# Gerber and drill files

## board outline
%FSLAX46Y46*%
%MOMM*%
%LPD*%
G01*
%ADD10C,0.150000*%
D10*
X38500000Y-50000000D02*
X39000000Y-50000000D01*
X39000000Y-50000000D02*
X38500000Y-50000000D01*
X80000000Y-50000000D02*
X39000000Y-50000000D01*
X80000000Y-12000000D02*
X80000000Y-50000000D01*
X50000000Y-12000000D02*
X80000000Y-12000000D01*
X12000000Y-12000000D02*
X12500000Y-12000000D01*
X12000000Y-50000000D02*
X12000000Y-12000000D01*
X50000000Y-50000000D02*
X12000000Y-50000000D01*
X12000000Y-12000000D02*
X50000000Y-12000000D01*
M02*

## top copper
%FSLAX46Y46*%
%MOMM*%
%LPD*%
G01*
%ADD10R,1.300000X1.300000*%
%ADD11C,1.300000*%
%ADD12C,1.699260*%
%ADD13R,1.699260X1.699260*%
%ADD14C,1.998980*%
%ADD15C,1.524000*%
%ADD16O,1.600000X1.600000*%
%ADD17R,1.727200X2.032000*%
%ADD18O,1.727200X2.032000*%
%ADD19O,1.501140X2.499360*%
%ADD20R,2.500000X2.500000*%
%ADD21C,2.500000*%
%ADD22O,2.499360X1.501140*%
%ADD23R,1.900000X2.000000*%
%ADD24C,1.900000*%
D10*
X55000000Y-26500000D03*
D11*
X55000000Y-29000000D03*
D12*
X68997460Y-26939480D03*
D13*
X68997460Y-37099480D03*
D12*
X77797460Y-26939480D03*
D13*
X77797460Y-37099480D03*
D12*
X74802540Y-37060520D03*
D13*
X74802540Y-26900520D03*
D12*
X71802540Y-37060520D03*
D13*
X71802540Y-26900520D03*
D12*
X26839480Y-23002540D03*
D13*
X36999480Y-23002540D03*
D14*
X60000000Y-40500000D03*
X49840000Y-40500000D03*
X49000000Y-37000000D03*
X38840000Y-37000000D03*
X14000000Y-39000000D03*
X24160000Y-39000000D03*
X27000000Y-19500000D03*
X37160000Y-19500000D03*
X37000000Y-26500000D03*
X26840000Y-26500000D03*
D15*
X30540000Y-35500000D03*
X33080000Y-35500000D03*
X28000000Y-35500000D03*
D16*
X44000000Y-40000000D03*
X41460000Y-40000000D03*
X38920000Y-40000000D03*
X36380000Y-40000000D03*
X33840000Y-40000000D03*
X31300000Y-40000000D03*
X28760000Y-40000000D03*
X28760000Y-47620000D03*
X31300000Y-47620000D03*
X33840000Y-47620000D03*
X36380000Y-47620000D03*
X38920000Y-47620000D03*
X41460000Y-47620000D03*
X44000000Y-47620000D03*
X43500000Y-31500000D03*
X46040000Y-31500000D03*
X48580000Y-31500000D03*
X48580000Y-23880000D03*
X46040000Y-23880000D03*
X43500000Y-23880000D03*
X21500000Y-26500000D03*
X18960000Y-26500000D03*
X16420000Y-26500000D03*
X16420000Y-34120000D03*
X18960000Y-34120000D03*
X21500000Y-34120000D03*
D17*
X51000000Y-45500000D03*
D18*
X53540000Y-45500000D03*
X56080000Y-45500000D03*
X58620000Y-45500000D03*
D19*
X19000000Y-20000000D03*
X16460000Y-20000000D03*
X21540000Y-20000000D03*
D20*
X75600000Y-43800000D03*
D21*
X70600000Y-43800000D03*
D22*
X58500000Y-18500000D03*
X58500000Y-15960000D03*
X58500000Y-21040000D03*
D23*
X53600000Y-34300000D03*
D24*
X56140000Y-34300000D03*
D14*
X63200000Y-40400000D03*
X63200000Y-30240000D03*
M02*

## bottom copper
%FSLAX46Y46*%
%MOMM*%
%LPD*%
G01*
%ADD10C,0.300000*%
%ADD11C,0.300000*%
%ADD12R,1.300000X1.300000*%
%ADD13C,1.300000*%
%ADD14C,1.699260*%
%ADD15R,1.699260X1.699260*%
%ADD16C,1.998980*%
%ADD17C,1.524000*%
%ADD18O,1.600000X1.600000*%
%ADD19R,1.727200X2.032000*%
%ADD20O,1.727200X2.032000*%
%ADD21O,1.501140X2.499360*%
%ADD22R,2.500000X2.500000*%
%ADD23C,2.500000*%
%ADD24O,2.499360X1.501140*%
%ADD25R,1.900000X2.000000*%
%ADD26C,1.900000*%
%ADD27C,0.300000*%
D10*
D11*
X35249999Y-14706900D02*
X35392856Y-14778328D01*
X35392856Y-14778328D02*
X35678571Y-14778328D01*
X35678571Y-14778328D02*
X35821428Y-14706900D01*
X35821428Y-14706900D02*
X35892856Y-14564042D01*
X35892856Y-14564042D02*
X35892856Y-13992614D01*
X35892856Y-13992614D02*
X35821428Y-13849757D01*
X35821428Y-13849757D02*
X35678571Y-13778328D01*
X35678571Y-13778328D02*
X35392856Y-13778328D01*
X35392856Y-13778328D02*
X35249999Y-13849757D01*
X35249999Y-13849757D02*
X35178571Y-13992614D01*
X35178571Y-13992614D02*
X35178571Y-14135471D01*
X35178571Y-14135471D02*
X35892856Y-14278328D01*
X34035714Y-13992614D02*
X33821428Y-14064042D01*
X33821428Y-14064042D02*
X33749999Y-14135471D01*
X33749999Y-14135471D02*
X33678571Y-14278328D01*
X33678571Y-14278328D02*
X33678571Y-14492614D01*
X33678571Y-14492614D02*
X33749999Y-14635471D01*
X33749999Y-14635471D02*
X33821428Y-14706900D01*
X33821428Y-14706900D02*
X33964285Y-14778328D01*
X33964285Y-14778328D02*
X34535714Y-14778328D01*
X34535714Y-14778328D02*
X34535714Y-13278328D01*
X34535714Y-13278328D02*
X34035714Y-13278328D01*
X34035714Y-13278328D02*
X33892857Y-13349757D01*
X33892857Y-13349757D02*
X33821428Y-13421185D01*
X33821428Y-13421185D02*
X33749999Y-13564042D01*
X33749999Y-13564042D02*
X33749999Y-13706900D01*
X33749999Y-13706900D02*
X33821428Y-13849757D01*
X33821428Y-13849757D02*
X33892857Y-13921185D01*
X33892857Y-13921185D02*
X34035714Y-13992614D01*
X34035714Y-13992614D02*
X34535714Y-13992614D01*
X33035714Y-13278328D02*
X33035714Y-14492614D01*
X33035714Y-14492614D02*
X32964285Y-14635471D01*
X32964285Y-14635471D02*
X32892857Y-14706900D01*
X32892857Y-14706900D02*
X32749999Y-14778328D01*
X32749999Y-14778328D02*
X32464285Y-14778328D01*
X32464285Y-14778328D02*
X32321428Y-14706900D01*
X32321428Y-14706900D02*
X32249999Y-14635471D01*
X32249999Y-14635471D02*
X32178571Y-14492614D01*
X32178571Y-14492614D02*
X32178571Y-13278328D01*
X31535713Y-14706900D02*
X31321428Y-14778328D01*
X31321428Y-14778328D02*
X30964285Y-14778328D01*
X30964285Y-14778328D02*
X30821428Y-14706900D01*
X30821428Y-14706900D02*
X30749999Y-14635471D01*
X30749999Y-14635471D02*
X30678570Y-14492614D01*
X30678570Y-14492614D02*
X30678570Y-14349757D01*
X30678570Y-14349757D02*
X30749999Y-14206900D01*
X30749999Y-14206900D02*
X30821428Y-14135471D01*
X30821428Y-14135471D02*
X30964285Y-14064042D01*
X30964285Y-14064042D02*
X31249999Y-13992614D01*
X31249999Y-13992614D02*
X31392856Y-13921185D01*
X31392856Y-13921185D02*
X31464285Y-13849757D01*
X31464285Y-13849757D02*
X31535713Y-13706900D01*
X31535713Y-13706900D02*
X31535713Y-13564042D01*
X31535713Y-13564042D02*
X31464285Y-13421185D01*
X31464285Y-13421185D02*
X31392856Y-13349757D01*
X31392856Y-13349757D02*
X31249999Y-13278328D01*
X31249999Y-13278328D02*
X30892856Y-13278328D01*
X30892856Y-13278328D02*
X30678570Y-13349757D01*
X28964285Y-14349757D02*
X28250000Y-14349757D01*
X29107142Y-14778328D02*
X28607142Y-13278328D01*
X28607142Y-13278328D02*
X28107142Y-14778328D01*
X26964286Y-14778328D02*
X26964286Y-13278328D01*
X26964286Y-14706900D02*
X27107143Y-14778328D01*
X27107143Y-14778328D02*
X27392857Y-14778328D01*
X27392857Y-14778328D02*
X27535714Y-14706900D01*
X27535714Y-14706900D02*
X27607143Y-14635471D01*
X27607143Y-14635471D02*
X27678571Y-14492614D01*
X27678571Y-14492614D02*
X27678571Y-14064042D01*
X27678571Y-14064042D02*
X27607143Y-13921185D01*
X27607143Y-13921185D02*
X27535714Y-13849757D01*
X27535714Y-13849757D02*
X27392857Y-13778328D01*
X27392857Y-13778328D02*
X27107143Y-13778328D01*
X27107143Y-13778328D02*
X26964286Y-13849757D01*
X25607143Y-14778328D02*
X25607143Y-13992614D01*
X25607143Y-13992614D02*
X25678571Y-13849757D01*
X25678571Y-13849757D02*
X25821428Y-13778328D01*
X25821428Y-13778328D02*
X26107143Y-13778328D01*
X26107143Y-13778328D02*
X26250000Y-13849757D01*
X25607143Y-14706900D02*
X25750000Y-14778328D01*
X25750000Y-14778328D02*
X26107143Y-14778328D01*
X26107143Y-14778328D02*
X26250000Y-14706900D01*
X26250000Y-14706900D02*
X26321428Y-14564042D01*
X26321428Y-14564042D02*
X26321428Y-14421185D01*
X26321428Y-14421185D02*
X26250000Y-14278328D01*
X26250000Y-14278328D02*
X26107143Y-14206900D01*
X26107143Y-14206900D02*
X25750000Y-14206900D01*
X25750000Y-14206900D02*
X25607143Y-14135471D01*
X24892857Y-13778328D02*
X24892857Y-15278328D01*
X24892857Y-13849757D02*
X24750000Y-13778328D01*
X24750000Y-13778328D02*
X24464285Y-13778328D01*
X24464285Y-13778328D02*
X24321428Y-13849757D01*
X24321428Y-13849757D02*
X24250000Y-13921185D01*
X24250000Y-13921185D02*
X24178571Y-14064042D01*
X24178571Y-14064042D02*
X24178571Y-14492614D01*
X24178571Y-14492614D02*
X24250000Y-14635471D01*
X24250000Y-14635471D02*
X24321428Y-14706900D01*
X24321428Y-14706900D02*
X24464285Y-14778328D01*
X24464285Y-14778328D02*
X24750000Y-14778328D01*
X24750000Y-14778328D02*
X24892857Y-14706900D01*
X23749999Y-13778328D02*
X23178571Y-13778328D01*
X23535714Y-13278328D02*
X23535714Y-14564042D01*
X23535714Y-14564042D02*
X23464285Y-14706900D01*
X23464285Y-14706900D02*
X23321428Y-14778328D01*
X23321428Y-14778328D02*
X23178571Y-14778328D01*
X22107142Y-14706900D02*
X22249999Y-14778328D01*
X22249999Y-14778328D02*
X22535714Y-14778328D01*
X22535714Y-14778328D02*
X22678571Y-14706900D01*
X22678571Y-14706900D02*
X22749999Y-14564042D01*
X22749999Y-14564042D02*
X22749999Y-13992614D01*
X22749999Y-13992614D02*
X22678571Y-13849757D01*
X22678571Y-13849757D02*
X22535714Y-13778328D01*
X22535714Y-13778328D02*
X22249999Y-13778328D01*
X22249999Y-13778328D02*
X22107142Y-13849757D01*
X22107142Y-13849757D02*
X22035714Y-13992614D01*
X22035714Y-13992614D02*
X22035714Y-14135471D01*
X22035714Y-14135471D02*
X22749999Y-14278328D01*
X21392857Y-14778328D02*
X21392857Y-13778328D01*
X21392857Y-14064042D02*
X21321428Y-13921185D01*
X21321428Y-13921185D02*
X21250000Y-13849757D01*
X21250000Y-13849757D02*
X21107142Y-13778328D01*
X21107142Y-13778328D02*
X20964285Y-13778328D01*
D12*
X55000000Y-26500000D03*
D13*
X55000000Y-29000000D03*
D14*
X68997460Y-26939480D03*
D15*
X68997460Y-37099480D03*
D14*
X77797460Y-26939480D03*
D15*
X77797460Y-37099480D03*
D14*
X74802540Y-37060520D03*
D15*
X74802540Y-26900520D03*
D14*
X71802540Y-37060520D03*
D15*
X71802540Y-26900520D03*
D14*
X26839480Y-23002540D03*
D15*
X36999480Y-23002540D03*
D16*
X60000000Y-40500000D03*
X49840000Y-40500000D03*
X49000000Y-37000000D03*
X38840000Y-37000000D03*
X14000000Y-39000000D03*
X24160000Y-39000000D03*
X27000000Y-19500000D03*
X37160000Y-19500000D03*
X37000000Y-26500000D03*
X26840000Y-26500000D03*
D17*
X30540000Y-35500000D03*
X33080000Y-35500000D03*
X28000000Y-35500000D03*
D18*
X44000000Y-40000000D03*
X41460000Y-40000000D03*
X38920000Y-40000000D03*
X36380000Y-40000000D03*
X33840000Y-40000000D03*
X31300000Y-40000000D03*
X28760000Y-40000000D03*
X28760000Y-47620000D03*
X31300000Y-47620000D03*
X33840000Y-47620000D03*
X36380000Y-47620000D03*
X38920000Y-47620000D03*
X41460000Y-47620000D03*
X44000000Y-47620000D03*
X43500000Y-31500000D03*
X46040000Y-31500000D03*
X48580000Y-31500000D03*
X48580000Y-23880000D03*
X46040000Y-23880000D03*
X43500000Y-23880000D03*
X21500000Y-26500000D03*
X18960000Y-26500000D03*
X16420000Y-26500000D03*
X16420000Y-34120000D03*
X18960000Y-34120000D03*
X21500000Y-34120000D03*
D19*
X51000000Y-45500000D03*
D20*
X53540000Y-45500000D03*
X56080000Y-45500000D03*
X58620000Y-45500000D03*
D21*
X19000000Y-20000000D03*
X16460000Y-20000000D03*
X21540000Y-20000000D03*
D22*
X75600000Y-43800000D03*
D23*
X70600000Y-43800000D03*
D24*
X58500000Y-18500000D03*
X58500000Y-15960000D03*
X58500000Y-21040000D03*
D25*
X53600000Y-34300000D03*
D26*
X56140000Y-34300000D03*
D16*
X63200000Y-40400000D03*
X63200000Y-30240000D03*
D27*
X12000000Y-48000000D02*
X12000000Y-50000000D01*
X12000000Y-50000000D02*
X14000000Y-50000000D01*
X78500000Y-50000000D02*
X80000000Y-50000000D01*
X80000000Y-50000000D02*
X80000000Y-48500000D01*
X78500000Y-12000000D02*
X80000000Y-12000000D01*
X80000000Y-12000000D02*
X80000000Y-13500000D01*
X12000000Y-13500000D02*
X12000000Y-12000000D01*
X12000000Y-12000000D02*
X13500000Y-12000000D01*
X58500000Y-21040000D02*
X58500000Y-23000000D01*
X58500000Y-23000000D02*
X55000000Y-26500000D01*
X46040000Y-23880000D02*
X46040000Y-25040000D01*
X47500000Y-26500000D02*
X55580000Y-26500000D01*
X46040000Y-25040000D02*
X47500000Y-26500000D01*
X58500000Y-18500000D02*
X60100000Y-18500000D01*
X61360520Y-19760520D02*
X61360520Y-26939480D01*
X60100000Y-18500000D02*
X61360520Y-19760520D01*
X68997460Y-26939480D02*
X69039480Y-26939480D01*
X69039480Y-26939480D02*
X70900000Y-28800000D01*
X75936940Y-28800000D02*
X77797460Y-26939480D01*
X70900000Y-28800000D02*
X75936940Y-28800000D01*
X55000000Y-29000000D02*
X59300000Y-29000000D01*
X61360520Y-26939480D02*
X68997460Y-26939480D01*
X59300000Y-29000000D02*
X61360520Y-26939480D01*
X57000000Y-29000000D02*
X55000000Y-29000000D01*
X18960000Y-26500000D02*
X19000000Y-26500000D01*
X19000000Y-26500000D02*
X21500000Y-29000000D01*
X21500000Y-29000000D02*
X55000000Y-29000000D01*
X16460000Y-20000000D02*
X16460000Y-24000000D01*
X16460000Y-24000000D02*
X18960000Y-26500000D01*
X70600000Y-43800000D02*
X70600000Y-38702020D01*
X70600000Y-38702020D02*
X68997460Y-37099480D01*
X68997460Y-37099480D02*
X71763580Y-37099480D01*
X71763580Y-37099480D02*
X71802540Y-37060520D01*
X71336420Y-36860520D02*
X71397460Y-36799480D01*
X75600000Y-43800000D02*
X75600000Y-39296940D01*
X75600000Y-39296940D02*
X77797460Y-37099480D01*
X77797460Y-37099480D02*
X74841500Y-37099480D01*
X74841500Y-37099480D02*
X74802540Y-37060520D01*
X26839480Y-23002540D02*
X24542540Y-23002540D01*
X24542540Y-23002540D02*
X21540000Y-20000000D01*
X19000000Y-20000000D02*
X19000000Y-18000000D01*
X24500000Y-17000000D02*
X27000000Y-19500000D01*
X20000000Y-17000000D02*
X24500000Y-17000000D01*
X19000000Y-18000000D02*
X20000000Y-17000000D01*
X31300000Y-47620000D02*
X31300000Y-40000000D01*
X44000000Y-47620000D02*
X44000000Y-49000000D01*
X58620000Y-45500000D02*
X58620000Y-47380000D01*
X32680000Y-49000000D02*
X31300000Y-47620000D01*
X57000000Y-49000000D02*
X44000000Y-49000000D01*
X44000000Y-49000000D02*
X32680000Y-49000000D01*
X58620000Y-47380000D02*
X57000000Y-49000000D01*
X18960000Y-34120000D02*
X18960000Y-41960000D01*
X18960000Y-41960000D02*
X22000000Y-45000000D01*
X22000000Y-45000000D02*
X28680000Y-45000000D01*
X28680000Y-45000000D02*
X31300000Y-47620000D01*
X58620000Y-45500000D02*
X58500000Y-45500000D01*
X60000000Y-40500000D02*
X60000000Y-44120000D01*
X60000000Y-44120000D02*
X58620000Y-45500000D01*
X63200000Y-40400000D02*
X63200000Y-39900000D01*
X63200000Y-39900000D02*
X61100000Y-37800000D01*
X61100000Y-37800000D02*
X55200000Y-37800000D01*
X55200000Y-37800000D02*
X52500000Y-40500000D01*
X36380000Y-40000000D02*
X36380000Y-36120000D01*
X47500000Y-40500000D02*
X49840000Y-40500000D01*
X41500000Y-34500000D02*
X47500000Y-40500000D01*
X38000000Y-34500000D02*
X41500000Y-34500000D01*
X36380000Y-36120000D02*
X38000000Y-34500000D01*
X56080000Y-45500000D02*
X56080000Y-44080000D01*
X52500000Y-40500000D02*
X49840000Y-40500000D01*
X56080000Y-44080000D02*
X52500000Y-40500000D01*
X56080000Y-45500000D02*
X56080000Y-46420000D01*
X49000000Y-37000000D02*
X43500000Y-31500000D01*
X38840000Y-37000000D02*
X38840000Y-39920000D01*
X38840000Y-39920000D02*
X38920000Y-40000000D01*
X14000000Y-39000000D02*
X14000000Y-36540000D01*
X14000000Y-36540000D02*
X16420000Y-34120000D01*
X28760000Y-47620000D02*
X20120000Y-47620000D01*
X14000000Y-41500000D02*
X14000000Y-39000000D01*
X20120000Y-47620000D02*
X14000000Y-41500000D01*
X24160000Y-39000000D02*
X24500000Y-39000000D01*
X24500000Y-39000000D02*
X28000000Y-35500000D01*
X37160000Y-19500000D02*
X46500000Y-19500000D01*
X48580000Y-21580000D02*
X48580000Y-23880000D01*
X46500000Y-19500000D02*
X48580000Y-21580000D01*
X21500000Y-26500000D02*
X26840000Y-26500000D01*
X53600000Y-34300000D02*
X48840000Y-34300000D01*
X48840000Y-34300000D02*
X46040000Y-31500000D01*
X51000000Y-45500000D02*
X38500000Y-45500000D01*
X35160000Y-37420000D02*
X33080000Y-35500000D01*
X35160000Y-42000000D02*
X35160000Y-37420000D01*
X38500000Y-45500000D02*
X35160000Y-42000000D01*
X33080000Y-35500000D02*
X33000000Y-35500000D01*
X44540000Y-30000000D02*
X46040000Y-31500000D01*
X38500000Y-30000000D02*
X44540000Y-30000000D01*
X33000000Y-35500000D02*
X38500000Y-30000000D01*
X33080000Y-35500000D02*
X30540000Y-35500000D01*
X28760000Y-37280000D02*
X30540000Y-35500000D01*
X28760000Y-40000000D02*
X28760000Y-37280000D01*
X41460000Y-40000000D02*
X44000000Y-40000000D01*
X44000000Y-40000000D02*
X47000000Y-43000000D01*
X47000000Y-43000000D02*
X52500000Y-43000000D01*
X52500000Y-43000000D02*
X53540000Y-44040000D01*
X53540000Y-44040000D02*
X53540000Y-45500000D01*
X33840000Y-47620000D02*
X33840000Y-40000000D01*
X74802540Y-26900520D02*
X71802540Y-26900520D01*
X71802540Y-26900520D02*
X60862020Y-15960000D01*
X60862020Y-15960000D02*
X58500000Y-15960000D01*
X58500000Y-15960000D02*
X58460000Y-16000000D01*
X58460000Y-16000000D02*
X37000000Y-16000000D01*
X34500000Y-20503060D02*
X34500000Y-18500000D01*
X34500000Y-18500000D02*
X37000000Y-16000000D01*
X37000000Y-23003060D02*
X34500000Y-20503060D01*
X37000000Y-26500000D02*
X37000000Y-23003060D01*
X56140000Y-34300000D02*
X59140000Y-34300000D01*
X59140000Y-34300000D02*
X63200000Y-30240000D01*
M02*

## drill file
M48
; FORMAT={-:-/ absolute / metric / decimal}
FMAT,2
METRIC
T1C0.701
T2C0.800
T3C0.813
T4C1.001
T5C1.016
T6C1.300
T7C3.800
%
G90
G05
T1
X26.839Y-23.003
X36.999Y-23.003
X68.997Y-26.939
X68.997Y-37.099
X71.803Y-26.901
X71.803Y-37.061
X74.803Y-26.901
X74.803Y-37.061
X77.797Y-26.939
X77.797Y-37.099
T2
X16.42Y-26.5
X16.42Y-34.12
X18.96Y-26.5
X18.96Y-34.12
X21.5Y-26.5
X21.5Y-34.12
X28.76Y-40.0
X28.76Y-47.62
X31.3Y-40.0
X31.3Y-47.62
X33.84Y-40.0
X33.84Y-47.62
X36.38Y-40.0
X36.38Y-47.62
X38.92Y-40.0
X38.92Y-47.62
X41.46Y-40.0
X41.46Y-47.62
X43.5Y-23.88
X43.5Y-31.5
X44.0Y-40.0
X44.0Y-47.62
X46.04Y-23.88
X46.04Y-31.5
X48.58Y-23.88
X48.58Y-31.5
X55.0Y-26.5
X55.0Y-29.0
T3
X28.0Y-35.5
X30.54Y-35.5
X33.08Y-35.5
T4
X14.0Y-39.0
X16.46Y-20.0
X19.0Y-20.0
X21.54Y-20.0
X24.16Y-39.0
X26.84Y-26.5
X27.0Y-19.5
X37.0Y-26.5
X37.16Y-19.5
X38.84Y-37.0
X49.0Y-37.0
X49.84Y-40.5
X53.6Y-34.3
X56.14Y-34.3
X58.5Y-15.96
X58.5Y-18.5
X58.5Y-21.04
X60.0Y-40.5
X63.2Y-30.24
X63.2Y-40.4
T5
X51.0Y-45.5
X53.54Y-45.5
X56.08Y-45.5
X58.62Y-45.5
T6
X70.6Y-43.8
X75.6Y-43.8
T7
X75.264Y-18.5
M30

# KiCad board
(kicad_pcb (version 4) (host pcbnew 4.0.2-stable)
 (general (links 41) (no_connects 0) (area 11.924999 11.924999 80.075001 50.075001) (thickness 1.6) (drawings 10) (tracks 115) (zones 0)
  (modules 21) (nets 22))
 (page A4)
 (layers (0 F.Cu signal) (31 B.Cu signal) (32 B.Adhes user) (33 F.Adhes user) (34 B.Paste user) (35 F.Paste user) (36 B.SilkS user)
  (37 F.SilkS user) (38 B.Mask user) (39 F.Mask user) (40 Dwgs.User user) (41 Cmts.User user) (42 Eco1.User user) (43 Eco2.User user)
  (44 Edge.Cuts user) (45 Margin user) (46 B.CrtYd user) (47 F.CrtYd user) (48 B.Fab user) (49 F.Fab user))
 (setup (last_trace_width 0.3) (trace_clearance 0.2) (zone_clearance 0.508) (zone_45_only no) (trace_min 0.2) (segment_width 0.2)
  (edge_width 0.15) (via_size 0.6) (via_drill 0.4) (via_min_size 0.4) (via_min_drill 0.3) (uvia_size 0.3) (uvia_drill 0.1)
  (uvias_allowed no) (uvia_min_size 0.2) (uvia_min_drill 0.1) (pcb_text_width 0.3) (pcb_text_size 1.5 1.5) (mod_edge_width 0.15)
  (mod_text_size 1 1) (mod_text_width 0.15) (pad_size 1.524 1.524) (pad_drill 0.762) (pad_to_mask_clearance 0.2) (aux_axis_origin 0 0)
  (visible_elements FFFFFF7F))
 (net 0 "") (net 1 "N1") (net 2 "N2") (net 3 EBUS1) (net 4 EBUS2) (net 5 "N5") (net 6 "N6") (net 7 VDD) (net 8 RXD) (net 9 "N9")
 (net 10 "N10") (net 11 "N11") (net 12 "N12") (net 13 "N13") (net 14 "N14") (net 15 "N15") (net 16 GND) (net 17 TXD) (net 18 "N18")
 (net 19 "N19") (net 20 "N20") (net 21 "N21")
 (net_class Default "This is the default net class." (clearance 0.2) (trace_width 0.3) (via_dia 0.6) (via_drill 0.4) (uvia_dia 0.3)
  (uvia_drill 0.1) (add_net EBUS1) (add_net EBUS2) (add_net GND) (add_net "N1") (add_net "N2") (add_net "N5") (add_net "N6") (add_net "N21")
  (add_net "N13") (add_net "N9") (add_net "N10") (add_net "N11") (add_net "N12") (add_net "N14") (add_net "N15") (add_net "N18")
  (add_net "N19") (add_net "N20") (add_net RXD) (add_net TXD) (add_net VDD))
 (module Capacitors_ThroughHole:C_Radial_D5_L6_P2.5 (layer F.Cu) (at 55 26.5 270)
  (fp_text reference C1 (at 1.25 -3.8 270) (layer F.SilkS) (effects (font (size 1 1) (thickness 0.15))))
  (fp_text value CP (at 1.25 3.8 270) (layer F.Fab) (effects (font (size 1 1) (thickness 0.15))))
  (pad 1 thru_hole rect (at 0 0 270) (size 1.3 1.3) (drill 0.8) (layers *.Cu *.Mask F.SilkS) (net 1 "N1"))
  (pad 2 thru_hole circle (at 2.5 0 270) (size 1.3 1.3) (drill 0.8) (layers *.Cu *.Mask F.SilkS) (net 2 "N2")))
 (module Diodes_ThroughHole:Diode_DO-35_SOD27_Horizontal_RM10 (layer F.Cu) (at 69 37.1 90)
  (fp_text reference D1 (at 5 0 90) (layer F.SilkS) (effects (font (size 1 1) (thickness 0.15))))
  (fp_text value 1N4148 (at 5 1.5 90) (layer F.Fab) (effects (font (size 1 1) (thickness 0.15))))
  (pad 2 thru_hole circle (at 10.16052 -0.00254 270) (size 1.69926 1.69926) (drill 0.70104) (layers *.Cu *.Mask F.SilkS) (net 2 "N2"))
  (pad 1 thru_hole rect (at 0.00052 -0.00254 270) (size 1.69926 1.69926) (drill 0.70104) (layers *.Cu *.Mask F.SilkS) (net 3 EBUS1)))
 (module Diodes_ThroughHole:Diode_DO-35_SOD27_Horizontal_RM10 (layer F.Cu) (at 77.8 37.1 90)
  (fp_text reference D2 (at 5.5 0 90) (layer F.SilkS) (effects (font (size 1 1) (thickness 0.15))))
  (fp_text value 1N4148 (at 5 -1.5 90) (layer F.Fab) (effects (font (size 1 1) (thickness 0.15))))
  (pad 2 thru_hole circle (at 10.16052 -0.00254 270) (size 1.69926 1.69926) (drill 0.70104) (layers *.Cu *.Mask F.SilkS) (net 2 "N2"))
  (pad 1 thru_hole rect (at 0.00052 -0.00254 270) (size 1.69926 1.69926) (drill 0.70104) (layers *.Cu *.Mask F.SilkS) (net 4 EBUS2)))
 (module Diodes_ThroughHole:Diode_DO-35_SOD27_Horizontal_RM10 (layer F.Cu) (at 74.8 26.9 270)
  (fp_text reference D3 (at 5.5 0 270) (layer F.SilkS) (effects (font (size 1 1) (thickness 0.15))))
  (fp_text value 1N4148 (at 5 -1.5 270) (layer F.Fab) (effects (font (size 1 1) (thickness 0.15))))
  (pad 2 thru_hole circle (at 10.16052 -0.00254 90) (size 1.69926 1.69926) (drill 0.70104) (layers *.Cu *.Mask F.SilkS) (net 4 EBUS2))
  (pad 1 thru_hole rect (at 0.00052 -0.00254 90) (size 1.69926 1.69926) (drill 0.70104) (layers *.Cu *.Mask F.SilkS) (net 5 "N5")))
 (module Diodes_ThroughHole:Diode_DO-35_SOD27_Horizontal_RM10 (layer F.Cu) (at 71.8 26.9 270)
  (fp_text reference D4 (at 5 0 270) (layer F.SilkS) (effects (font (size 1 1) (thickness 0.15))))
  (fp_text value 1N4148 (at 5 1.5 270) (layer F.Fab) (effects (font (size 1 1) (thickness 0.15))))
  (pad 2 thru_hole circle (at 10.16052 -0.00254 90) (size 1.69926 1.69926) (drill 0.70104) (layers *.Cu *.Mask F.SilkS) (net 3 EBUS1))
  (pad 1 thru_hole rect (at 0.00052 -0.00254 90) (size 1.69926 1.69926) (drill 0.70104) (layers *.Cu *.Mask F.SilkS) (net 5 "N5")))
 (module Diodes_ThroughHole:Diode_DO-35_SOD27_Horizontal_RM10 (layer F.Cu) (at 37 23 180)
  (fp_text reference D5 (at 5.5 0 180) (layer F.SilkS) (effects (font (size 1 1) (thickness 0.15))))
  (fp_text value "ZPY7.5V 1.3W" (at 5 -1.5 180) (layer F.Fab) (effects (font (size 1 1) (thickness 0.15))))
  (pad 2 thru_hole circle (at 10.16052 -0.00254) (size 1.69926 1.69926) (drill 0.70104) (layers *.Cu *.Mask F.SilkS) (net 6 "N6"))
  (pad 1 thru_hole rect (at 0.00052 -0.00254) (size 1.69926 1.69926) (drill 0.70104) (layers *.Cu *.Mask F.SilkS) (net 5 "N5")))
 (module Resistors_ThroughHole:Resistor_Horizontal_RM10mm (layer F.Cu) (at 60 40.5 180)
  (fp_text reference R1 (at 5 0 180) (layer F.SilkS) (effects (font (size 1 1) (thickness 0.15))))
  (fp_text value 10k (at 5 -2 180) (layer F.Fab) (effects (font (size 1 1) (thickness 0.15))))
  (pad 1 thru_hole circle (at 0 0 180) (size 1.99898 1.99898) (drill 1.00076) (layers *.Cu *.SilkS *.Mask) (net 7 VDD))
  (pad 2 thru_hole circle (at 10.16 0 180) (size 1.99898 1.99898) (drill 1.00076) (layers *.Cu *.SilkS *.Mask) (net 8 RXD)))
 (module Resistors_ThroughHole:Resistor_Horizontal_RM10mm (layer F.Cu) (at 49 37 180)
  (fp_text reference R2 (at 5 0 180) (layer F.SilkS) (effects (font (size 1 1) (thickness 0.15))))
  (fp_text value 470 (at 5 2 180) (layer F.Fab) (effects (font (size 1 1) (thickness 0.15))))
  (pad 1 thru_hole circle (at 0 0 180) (size 1.99898 1.99898) (drill 1.00076) (layers *.Cu *.SilkS *.Mask) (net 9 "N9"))
  (pad 2 thru_hole circle (at 10.16 0 180) (size 1.99898 1.99898) (drill 1.00076) (layers *.Cu *.SilkS *.Mask) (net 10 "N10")))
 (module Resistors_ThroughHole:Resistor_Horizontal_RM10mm (layer F.Cu) (at 14 39)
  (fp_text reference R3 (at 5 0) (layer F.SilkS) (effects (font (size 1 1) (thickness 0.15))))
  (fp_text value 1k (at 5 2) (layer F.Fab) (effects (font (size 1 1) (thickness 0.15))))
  (pad 1 thru_hole circle (at 0 0) (size 1.99898 1.99898) (drill 1.00076) (layers *.Cu *.SilkS *.Mask) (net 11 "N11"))
  (pad 2 thru_hole circle (at 10.16 0) (size 1.99898 1.99898) (drill 1.00076) (layers *.Cu *.SilkS *.Mask) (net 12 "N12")))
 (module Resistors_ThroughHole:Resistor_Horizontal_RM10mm (layer F.Cu) (at 27 19.5)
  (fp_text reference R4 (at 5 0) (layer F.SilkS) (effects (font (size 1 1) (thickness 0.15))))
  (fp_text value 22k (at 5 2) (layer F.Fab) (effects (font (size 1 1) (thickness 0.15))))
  (pad 1 thru_hole circle (at 0 0) (size 1.99898 1.99898) (drill 1.00076) (layers *.Cu *.SilkS *.Mask) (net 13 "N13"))
  (pad 2 thru_hole circle (at 10.16 0) (size 1.99898 1.99898) (drill 1.00076) (layers *.Cu *.SilkS *.Mask) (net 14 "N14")))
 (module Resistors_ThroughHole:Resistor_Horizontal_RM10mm (layer F.Cu) (at 37 26.5 180)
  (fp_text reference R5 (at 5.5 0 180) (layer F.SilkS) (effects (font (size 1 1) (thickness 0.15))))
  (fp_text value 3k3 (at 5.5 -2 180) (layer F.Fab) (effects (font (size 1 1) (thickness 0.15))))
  (pad 1 thru_hole circle (at 0 0 180) (size 1.99898 1.99898) (drill 1.00076) (layers *.Cu *.SilkS *.Mask) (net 5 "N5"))
  (pad 2 thru_hole circle (at 10.16 0 180) (size 1.99898 1.99898) (drill 1.00076) (layers *.Cu *.SilkS *.Mask) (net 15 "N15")))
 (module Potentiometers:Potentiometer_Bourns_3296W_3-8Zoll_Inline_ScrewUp (layer F.Cu) (at 28 35.5 270)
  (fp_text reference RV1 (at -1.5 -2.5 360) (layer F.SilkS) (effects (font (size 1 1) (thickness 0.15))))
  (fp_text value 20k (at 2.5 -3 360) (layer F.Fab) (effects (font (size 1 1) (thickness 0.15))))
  (pad 2 thru_hole circle (at 0 -2.54 270) (size 1.524 1.524) (drill 0.8128) (layers *.Cu *.Mask F.SilkS) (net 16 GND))
  (pad 3 thru_hole circle (at 0 -5.08 270) (size 1.524 1.524) (drill 0.8128) (layers *.Cu *.Mask F.SilkS) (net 16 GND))
  (pad 1 thru_hole circle (at 0 0 270) (size 1.524 1.524) (drill 0.8128) (layers *.Cu *.Mask F.SilkS) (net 12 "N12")))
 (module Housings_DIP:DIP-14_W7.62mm (layer F.Cu) (at 44 40 270)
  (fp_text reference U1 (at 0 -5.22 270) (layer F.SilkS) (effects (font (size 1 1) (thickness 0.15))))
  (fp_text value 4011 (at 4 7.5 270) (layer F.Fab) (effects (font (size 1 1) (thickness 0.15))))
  (pad 1 thru_hole oval (at 0 0 270) (size 1.6 1.6) (drill 0.8) (layers *.Cu *.Mask F.SilkS) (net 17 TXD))
  (pad 2 thru_hole oval (at 0 2.54 270) (size 1.6 1.6) (drill 0.8) (layers *.Cu *.Mask F.SilkS) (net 17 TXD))
  (pad 3 thru_hole oval (at 0 5.08 270) (size 1.6 1.6) (drill 0.8) (layers *.Cu *.Mask F.SilkS) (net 10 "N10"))
  (pad 4 thru_hole oval (at 0 7.62 270) (size 1.6 1.6) (drill 0.8) (layers *.Cu *.Mask F.SilkS) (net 8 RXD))
  (pad 5 thru_hole oval (at 0 10.16 270) (size 1.6 1.6) (drill 0.8) (layers *.Cu *.Mask F.SilkS) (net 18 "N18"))
  (pad 6 thru_hole oval (at 0 12.7 270) (size 1.6 1.6) (drill 0.8) (layers *.Cu *.Mask F.SilkS) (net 7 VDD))
  (pad 7 thru_hole oval (at 0 15.24 270) (size 1.6 1.6) (drill 0.8) (layers *.Cu *.Mask F.SilkS) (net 16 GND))
  (pad 8 thru_hole oval (at 7.62 15.24 270) (size 1.6 1.6) (drill 0.8) (layers *.Cu *.Mask F.SilkS) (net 11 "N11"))
  (pad 9 thru_hole oval (at 7.62 12.7 270) (size 1.6 1.6) (drill 0.8) (layers *.Cu *.Mask F.SilkS) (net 7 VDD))
  (pad 10 thru_hole oval (at 7.62 10.16 270) (size 1.6 1.6) (drill 0.8) (layers *.Cu *.Mask F.SilkS) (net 18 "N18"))
  (pad 11 thru_hole oval (at 7.62 7.62 270) (size 1.6 1.6) (drill 0.8) (layers *.Cu *.Mask F.SilkS))
  (pad 12 thru_hole oval (at 7.62 5.08 270) (size 1.6 1.6) (drill 0.8) (layers *.Cu *.Mask F.SilkS))
  (pad 13 thru_hole oval (at 7.62 2.54 270) (size 1.6 1.6) (drill 0.8) (layers *.Cu *.Mask F.SilkS))
  (pad 14 thru_hole oval (at 7.62 0 270) (size 1.6 1.6) (drill 0.8) (layers *.Cu *.Mask F.SilkS) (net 7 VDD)))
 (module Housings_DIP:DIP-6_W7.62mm (layer F.Cu) (at 43.5 31.5 90)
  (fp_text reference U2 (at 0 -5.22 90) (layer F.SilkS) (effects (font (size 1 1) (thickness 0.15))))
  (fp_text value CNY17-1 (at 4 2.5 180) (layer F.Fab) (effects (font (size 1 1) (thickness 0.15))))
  (pad 1 thru_hole oval (at 0 0 90) (size 1.6 1.6) (drill 0.8) (layers *.Cu *.Mask F.SilkS) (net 9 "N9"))
  (pad 2 thru_hole oval (at 0 2.54 90) (size 1.6 1.6) (drill 0.8) (layers *.Cu *.Mask F.SilkS) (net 16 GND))
  (pad 3 thru_hole oval (at 0 5.08 90) (size 1.6 1.6) (drill 0.8) (layers *.Cu *.Mask F.SilkS))
  (pad 4 thru_hole oval (at 7.62 5.08 90) (size 1.6 1.6) (drill 0.8) (layers *.Cu *.Mask F.SilkS) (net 14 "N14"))
  (pad 5 thru_hole oval (at 7.62 2.54 90) (size 1.6 1.6) (drill 0.8) (layers *.Cu *.Mask F.SilkS) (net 1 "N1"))
  (pad 6 thru_hole oval (at 7.62 0 90) (size 1.6 1.6) (drill 0.8) (layers *.Cu *.Mask F.SilkS) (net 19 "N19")))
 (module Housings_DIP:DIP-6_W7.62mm (layer F.Cu) (at 21.5 26.5 270)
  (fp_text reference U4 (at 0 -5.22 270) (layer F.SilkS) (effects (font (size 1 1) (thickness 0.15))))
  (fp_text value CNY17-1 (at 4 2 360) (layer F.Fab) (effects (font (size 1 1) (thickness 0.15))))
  (pad 1 thru_hole oval (at 0 0 270) (size 1.6 1.6) (drill 0.8) (layers *.Cu *.Mask F.SilkS) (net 15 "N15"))
  (pad 2 thru_hole oval (at 0 2.54 270) (size 1.6 1.6) (drill 0.8) (layers *.Cu *.Mask F.SilkS) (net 2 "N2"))
  (pad 3 thru_hole oval (at 0 5.08 270) (size 1.6 1.6) (drill 0.8) (layers *.Cu *.Mask F.SilkS))
  (pad 4 thru_hole oval (at 7.62 5.08 270) (size 1.6 1.6) (drill 0.8) (layers *.Cu *.Mask F.SilkS) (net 11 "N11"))
  (pad 5 thru_hole oval (at 7.62 2.54 270) (size 1.6 1.6) (drill 0.8) (layers *.Cu *.Mask F.SilkS) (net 7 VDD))
  (pad 6 thru_hole oval (at 7.62 0 270) (size 1.6 1.6) (drill 0.8) (layers *.Cu *.Mask F.SilkS) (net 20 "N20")))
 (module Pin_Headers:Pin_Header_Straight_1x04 (layer F.Cu) (at 51 45.5 90)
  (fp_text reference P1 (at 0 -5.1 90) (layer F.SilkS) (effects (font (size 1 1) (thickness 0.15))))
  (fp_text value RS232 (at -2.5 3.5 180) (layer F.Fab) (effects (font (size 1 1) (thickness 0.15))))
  (pad 1 thru_hole rect (at 0 0 90) (size 2.032 1.7272) (drill 1.016) (layers *.Cu *.Mask F.SilkS) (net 16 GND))
  (pad 2 thru_hole oval (at 0 2.54 90) (size 2.032 1.7272) (drill 1.016) (layers *.Cu *.Mask F.SilkS) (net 17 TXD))
  (pad 3 thru_hole oval (at 0 5.08 90) (size 2.032 1.7272) (drill 1.016) (layers *.Cu *.Mask F.SilkS) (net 8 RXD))
  (pad 4 thru_hole oval (at 0 7.62 90) (size 2.032 1.7272) (drill 1.016) (layers *.Cu *.Mask F.SilkS) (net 7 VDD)))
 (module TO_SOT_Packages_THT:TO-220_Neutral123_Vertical (layer F.Cu) (at 19 20)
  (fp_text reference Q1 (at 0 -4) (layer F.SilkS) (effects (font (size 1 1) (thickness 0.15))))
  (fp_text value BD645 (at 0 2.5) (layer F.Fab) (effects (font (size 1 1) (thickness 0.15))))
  (pad 2 thru_hole oval (at 0 0 90) (size 2.49936 1.50114) (drill 1.00076) (layers *.Cu *.Mask F.SilkS) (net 13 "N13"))
  (pad 1 thru_hole oval (at -2.54 0 90) (size 2.49936 1.50114) (drill 1.00076) (layers *.Cu *.Mask F.SilkS) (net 2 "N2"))
  (pad 3 thru_hole oval (at 2.54 0 90) (size 2.49936 1.50114) (drill 1.00076) (layers *.Cu *.Mask F.SilkS) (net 6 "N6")))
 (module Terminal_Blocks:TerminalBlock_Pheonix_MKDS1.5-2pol (layer F.Cu) (at 75.6 43.8 180)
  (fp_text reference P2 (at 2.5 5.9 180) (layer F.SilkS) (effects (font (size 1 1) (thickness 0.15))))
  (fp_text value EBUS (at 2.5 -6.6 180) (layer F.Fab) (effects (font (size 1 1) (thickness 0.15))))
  (pad 1 thru_hole rect (at 0 0 180) (size 2.5 2.5) (drill 1.3) (layers *.Cu *.Mask F.SilkS) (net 4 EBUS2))
  (pad 2 thru_hole circle (at 5 0 180) (size 2.5 2.5) (drill 1.3) (layers *.Cu *.Mask F.SilkS) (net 3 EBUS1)))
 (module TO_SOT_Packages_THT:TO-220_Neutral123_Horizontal (layer F.Cu) (at 58.5 18.5 270)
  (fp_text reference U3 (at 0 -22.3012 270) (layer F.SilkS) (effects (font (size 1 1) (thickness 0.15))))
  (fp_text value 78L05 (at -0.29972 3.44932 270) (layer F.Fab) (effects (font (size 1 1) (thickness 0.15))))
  (pad 2 thru_hole oval (at 0 0) (size 2.49936 1.50114) (drill 1.00076) (layers *.Cu *.Mask F.SilkS) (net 2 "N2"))
  (pad 1 thru_hole oval (at -2.54 0) (size 2.49936 1.50114) (drill 1.00076) (layers *.Cu *.Mask F.SilkS) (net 5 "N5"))
  (pad 3 thru_hole oval (at 2.54 0) (size 2.49936 1.50114) (drill 1.00076) (layers *.Cu *.Mask F.SilkS) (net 1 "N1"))
  (pad "" np_thru_hole circle (at 0 -16.764) (size 3.79984 3.79984) (drill 3.79984) (layers *.Cu *.Mask F.SilkS)))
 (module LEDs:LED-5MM (layer F.Cu) (at 53.6 34.3)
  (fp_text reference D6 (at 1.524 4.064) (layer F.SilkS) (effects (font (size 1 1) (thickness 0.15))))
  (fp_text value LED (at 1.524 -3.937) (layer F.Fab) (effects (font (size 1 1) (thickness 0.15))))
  (pad 1 thru_hole rect (at 0 0 90) (size 2 1.9) (drill 1.00076) (layers *.Cu *.Mask F.SilkS) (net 16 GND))
  (pad 2 thru_hole circle (at 2.54 0) (size 1.9 1.9) (drill 1.00076) (layers *.Cu *.Mask F.SilkS) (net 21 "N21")))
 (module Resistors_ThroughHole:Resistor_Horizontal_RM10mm (layer F.Cu) (at 63.2 40.4 90)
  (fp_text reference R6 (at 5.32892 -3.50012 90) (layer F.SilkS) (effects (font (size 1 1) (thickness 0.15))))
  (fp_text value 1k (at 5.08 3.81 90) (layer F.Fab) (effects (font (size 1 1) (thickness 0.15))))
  (pad 1 thru_hole circle (at 0 0 90) (size 1.99898 1.99898) (drill 1.00076) (layers *.Cu *.SilkS *.Mask) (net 8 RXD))
  (pad 2 thru_hole circle (at 10.16 0 90) (size 1.99898 1.99898) (drill 1.00076) (layers *.Cu *.SilkS *.Mask) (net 21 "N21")))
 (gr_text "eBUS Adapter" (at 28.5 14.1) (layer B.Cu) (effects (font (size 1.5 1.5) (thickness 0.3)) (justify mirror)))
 (gr_line (start 38.5 50) (end 39 50) (angle 90) (layer Edge.Cuts) (width 0.15))
 (gr_line (start 39 50) (end 38.5 50) (angle 90) (layer Edge.Cuts) (width 0.15))
 (gr_line (start 80 50) (end 39 50) (angle 90) (layer Edge.Cuts) (width 0.15))
 (gr_line (start 80 12) (end 80 50) (angle 90) (layer Edge.Cuts) (width 0.15))
 (gr_line (start 50 12) (end 80 12) (angle 90) (layer Edge.Cuts) (width 0.15))
 (gr_line (start 12 12) (end 12.5 12) (angle 90) (layer Edge.Cuts) (width 0.15))
 (gr_line (start 12 50) (end 12 12) (angle 90) (layer Edge.Cuts) (width 0.15))
 (gr_line (start 50 50) (end 12 50) (angle 90) (layer Edge.Cuts) (width 0.15))
 (gr_line (start 12 12) (end 50 12) (angle 90) (layer Edge.Cuts) (width 0.15))
 (segment (start 12 48) (end 12 50) (width 0.3) (layer B.Cu) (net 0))
 (segment (start 12 50) (end 14 50) (width 0.3) (layer B.Cu) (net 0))
 (segment (start 78.5 50) (end 80 50) (width 0.3) (layer B.Cu) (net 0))
 (segment (start 80 50) (end 80 48.5) (width 0.3) (layer B.Cu) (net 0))
 (segment (start 78.5 12) (end 80 12) (width 0.3) (layer B.Cu) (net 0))
 (segment (start 80 12) (end 80 13.5) (width 0.3) (layer B.Cu) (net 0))
 (segment (start 12 13.5) (end 12 12) (width 0.3) (layer B.Cu) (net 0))
 (segment (start 12 12) (end 13.5 12) (width 0.3) (layer B.Cu) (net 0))
 (segment (start 58.5 21.04) (end 58.5 23) (width 0.3) (layer B.Cu) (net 1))
 (segment (start 58.5 23) (end 55 26.5) (width 0.3) (layer B.Cu) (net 1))
 (segment (start 46.04 23.88) (end 46.04 25.04) (width 0.3) (layer B.Cu) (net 1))
 (segment (start 47.5 26.5) (end 55.58 26.5) (width 0.3) (layer B.Cu) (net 1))
 (segment (start 46.04 25.04) (end 47.5 26.5) (width 0.3) (layer B.Cu) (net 1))
 (segment (start 58.5 18.5) (end 60.1 18.5) (width 0.3) (layer B.Cu) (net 2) (status 400000))
 (segment (start 61.36052 19.76052) (end 61.36052 26.93948) (width 0.3) (layer B.Cu) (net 2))
 (segment (start 60.1 18.5) (end 61.36052 19.76052) (width 0.3) (layer B.Cu) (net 2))
 (segment (start 68.99746 26.93948) (end 69.03948 26.93948) (width 0.3) (layer B.Cu) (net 2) (status C00000))
 (segment (start 69.03948 26.93948) (end 70.9 28.8) (width 0.3) (layer B.Cu) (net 2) (status 400000))
 (segment (start 75.93694 28.8) (end 77.79746 26.93948) (width 0.3) (layer B.Cu) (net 2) (status 800000))
 (segment (start 70.9 28.8) (end 75.93694 28.8) (width 0.3) (layer B.Cu) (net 2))
 (segment (start 55 29) (end 59.3 29) (width 0.3) (layer B.Cu) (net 2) (status 400000))
 (segment (start 61.36052 26.93948) (end 68.99746 26.93948) (width 0.3) (layer B.Cu) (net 2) (status 800000))
 (segment (start 59.3 29) (end 61.36052 26.93948) (width 0.3) (layer B.Cu) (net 2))
 (segment (start 57 29) (end 55 29) (width 0.3) (layer B.Cu) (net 2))
 (segment (start 18.96 26.5) (end 19 26.5) (width 0.3) (layer B.Cu) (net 2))
 (segment (start 19 26.5) (end 21.5 29) (width 0.3) (layer B.Cu) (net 2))
 (segment (start 21.5 29) (end 55 29) (width 0.3) (layer B.Cu) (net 2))
 (segment (start 16.46 20) (end 16.46 24) (width 0.3) (layer B.Cu) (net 2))
 (segment (start 16.46 24) (end 18.96 26.5) (width 0.3) (layer B.Cu) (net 2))
 (segment (start 70.6 43.8) (end 70.6 38.70202) (width 0.3) (layer B.Cu) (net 3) (status 400000))
 (segment (start 70.6 38.70202) (end 68.99746 37.09948) (width 0.3) (layer B.Cu) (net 3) (status 800000))
 (segment (start 68.99746 37.09948) (end 71.76358 37.09948) (width 0.3) (layer B.Cu) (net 3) (status C00000))
 (segment (start 71.76358 37.09948) (end 71.80254 37.06052) (width 0.3) (layer B.Cu) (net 3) (status C00000))
 (segment (start 71.33642 36.86052) (end 71.39746 36.79948) (width 0.3) (layer B.Cu) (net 3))
 (segment (start 75.6 43.8) (end 75.6 39.29694) (width 0.3) (layer B.Cu) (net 4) (status 400000))
 (segment (start 75.6 39.29694) (end 77.79746 37.09948) (width 0.3) (layer B.Cu) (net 4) (status 800000))
 (segment (start 77.79746 37.09948) (end 74.8415 37.09948) (width 0.3) (layer B.Cu) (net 4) (status C00000))
 (segment (start 74.8415 37.09948) (end 74.80254 37.06052) (width 0.3) (layer B.Cu) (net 4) (status C00000))
 (segment (start 26.83948 23.00254) (end 24.54254 23.00254) (width 0.3) (layer B.Cu) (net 6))
 (segment (start 24.54254 23.00254) (end 21.54 20) (width 0.3) (layer B.Cu) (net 6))
 (segment (start 19 20) (end 19 18) (width 0.3) (layer B.Cu) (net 13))
 (segment (start 24.5 17) (end 27 19.5) (width 0.3) (layer B.Cu) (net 13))
 (segment (start 20 17) (end 24.5 17) (width 0.3) (layer B.Cu) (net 13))
 (segment (start 19 18) (end 20 17) (width 0.3) (layer B.Cu) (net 13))
 (segment (start 31.3 47.62) (end 31.3 40) (width 0.3) (layer B.Cu) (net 7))
 (segment (start 44 47.62) (end 44 49) (width 0.3) (layer B.Cu) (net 7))
 (segment (start 58.62 45.5) (end 58.62 47.38) (width 0.3) (layer B.Cu) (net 7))
 (segment (start 32.68 49) (end 31.3 47.62) (width 0.3) (layer B.Cu) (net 7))
 (segment (start 57 49) (end 44 49) (width 0.3) (layer B.Cu) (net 7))
 (segment (start 44 49) (end 32.68 49) (width 0.3) (layer B.Cu) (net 7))
 (segment (start 58.62 47.38) (end 57 49) (width 0.3) (layer B.Cu) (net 7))
 (segment (start 18.96 34.12) (end 18.96 41.96) (width 0.3) (layer B.Cu) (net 7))
 (segment (start 18.96 41.96) (end 22 45) (width 0.3) (layer B.Cu) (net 7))
 (segment (start 22 45) (end 28.68 45) (width 0.3) (layer B.Cu) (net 7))
 (segment (start 28.68 45) (end 31.3 47.62) (width 0.3) (layer B.Cu) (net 7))
 (segment (start 58.62 45.5) (end 58.5 45.5) (width 0.3) (layer B.Cu) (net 7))
 (segment (start 60 40.5) (end 60 44.12) (width 0.3) (layer B.Cu) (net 7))
 (segment (start 60 44.12) (end 58.62 45.5) (width 0.3) (layer B.Cu) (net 7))
 (segment (start 63.2 40.4) (end 63.2 39.9) (width 0.3) (layer B.Cu) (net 8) (status C00000))
 (segment (start 63.2 39.9) (end 61.1 37.8) (width 0.3) (layer B.Cu) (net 8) (status 400000))
 (segment (start 61.1 37.8) (end 55.2 37.8) (width 0.3) (layer B.Cu) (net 8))
 (segment (start 55.2 37.8) (end 52.5 40.5) (width 0.3) (layer B.Cu) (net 8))
 (segment (start 36.38 40) (end 36.38 36.12) (width 0.3) (layer B.Cu) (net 8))
 (segment (start 47.5 40.5) (end 49.84 40.5) (width 0.3) (layer B.Cu) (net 8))
 (segment (start 41.5 34.5) (end 47.5 40.5) (width 0.3) (layer B.Cu) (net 8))
 (segment (start 38 34.5) (end 41.5 34.5) (width 0.3) (layer B.Cu) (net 8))
 (segment (start 36.38 36.12) (end 38 34.5) (width 0.3) (layer B.Cu) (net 8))
 (segment (start 56.08 45.5) (end 56.08 44.08) (width 0.3) (layer B.Cu) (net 8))
 (segment (start 52.5 40.5) (end 49.84 40.5) (width 0.3) (layer B.Cu) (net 8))
 (segment (start 56.08 44.08) (end 52.5 40.5) (width 0.3) (layer B.Cu) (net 8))
 (segment (start 56.08 45.5) (end 56.08 46.42) (width 0.3) (layer B.Cu) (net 8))
 (segment (start 49 37) (end 43.5 31.5) (width 0.3) (layer B.Cu) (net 9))
 (segment (start 38.84 37) (end 38.84 39.92) (width 0.3) (layer B.Cu) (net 10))
 (segment (start 38.84 39.92) (end 38.92 40) (width 0.3) (layer B.Cu) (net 10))
 (segment (start 14 39) (end 14 36.54) (width 0.3) (layer B.Cu) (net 11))
 (segment (start 14 36.54) (end 16.42 34.12) (width 0.3) (layer B.Cu) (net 11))
 (segment (start 28.76 47.62) (end 20.12 47.62) (width 0.3) (layer B.Cu) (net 11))
 (segment (start 14 41.5) (end 14 39) (width 0.3) (layer B.Cu) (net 11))
 (segment (start 20.12 47.62) (end 14 41.5) (width 0.3) (layer B.Cu) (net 11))
 (segment (start 24.16 39) (end 24.5 39) (width 0.3) (layer B.Cu) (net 12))
 (segment (start 24.5 39) (end 28 35.5) (width 0.3) (layer B.Cu) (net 12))
 (segment (start 37.16 19.5) (end 46.5 19.5) (width 0.3) (layer B.Cu) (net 14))
 (segment (start 48.58 21.58) (end 48.58 23.88) (width 0.3) (layer B.Cu) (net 14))
 (segment (start 46.5 19.5) (end 48.58 21.58) (width 0.3) (layer B.Cu) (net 14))
 (segment (start 21.5 26.5) (end 26.84 26.5) (width 0.3) (layer B.Cu) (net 15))
 (segment (start 53.6 34.3) (end 48.84 34.3) (width 0.3) (layer B.Cu) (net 16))
 (segment (start 48.84 34.3) (end 46.04 31.5) (width 0.3) (layer B.Cu) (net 16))
 (segment (start 51 45.5) (end 38.5 45.5) (width 0.3) (layer B.Cu) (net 16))
 (segment (start 35.16 37.42) (end 33.08 35.5) (width 0.3) (layer B.Cu) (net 16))
 (segment (start 35.16 42) (end 35.16 37.42) (width 0.3) (layer B.Cu) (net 16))
 (segment (start 38.5 45.5) (end 35.16 42) (width 0.3) (layer B.Cu) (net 16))
 (segment (start 33.08 35.5) (end 33 35.5) (width 0.3) (layer B.Cu) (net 16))
 (segment (start 44.54 30) (end 46.04 31.5) (width 0.3) (layer B.Cu) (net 16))
 (segment (start 38.5 30) (end 44.54 30) (width 0.3) (layer B.Cu) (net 16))
 (segment (start 33 35.5) (end 38.5 30) (width 0.3) (layer B.Cu) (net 16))
 (segment (start 33.08 35.5) (end 30.54 35.5) (width 0.3) (layer B.Cu) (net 16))
 (segment (start 28.76 37.28) (end 30.54 35.5) (width 0.3) (layer B.Cu) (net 16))
 (segment (start 28.76 40) (end 28.76 37.28) (width 0.3) (layer B.Cu) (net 16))
 (segment (start 41.46 40) (end 44 40) (width 0.3) (layer B.Cu) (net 17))
 (segment (start 44 40) (end 47 43) (width 0.3) (layer B.Cu) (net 17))
 (segment (start 47 43) (end 52.5 43) (width 0.3) (layer B.Cu) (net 17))
 (segment (start 52.5 43) (end 53.54 44.04) (width 0.3) (layer B.Cu) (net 17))
 (segment (start 53.54 44.04) (end 53.54 45.5) (width 0.3) (layer B.Cu) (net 17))
 (segment (start 33.84 47.62) (end 33.84 40) (width 0.3) (layer B.Cu) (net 18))
 (segment (start 74.80254 26.90052) (end 71.80254 26.90052) (width 0.3) (layer B.Cu) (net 5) (status C00000))
 (segment (start 71.80254 26.90052) (end 60.86202 15.96) (width 0.3) (layer B.Cu) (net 5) (status 400000))
 (segment (start 60.86202 15.96) (end 58.5 15.96) (width 0.3) (layer B.Cu) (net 5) (status 800000))
 (segment (start 58.5 15.96) (end 58.46 16) (width 0.3) (layer B.Cu) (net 5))
 (segment (start 58.46 16) (end 37 16) (width 0.3) (layer B.Cu) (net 5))
 (segment (start 34.5 20.50306) (end 34.5 18.5) (width 0.3) (layer B.Cu) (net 5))
 (segment (start 34.5 18.5) (end 37 16) (width 0.3) (layer B.Cu) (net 5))
 (segment (start 37 23.00306) (end 34.5 20.50306) (width 0.3) (layer B.Cu) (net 5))
 (segment (start 37 26.5) (end 37 23.00306) (width 0.3) (layer B.Cu) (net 5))
 (segment (start 56.14 34.3) (end 59.14 34.3) (width 0.3) (layer B.Cu) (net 21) (status 400000))
 (segment (start 59.14 34.3) (end 63.2 30.24) (width 0.3) (layer B.Cu) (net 21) (status 800000)))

